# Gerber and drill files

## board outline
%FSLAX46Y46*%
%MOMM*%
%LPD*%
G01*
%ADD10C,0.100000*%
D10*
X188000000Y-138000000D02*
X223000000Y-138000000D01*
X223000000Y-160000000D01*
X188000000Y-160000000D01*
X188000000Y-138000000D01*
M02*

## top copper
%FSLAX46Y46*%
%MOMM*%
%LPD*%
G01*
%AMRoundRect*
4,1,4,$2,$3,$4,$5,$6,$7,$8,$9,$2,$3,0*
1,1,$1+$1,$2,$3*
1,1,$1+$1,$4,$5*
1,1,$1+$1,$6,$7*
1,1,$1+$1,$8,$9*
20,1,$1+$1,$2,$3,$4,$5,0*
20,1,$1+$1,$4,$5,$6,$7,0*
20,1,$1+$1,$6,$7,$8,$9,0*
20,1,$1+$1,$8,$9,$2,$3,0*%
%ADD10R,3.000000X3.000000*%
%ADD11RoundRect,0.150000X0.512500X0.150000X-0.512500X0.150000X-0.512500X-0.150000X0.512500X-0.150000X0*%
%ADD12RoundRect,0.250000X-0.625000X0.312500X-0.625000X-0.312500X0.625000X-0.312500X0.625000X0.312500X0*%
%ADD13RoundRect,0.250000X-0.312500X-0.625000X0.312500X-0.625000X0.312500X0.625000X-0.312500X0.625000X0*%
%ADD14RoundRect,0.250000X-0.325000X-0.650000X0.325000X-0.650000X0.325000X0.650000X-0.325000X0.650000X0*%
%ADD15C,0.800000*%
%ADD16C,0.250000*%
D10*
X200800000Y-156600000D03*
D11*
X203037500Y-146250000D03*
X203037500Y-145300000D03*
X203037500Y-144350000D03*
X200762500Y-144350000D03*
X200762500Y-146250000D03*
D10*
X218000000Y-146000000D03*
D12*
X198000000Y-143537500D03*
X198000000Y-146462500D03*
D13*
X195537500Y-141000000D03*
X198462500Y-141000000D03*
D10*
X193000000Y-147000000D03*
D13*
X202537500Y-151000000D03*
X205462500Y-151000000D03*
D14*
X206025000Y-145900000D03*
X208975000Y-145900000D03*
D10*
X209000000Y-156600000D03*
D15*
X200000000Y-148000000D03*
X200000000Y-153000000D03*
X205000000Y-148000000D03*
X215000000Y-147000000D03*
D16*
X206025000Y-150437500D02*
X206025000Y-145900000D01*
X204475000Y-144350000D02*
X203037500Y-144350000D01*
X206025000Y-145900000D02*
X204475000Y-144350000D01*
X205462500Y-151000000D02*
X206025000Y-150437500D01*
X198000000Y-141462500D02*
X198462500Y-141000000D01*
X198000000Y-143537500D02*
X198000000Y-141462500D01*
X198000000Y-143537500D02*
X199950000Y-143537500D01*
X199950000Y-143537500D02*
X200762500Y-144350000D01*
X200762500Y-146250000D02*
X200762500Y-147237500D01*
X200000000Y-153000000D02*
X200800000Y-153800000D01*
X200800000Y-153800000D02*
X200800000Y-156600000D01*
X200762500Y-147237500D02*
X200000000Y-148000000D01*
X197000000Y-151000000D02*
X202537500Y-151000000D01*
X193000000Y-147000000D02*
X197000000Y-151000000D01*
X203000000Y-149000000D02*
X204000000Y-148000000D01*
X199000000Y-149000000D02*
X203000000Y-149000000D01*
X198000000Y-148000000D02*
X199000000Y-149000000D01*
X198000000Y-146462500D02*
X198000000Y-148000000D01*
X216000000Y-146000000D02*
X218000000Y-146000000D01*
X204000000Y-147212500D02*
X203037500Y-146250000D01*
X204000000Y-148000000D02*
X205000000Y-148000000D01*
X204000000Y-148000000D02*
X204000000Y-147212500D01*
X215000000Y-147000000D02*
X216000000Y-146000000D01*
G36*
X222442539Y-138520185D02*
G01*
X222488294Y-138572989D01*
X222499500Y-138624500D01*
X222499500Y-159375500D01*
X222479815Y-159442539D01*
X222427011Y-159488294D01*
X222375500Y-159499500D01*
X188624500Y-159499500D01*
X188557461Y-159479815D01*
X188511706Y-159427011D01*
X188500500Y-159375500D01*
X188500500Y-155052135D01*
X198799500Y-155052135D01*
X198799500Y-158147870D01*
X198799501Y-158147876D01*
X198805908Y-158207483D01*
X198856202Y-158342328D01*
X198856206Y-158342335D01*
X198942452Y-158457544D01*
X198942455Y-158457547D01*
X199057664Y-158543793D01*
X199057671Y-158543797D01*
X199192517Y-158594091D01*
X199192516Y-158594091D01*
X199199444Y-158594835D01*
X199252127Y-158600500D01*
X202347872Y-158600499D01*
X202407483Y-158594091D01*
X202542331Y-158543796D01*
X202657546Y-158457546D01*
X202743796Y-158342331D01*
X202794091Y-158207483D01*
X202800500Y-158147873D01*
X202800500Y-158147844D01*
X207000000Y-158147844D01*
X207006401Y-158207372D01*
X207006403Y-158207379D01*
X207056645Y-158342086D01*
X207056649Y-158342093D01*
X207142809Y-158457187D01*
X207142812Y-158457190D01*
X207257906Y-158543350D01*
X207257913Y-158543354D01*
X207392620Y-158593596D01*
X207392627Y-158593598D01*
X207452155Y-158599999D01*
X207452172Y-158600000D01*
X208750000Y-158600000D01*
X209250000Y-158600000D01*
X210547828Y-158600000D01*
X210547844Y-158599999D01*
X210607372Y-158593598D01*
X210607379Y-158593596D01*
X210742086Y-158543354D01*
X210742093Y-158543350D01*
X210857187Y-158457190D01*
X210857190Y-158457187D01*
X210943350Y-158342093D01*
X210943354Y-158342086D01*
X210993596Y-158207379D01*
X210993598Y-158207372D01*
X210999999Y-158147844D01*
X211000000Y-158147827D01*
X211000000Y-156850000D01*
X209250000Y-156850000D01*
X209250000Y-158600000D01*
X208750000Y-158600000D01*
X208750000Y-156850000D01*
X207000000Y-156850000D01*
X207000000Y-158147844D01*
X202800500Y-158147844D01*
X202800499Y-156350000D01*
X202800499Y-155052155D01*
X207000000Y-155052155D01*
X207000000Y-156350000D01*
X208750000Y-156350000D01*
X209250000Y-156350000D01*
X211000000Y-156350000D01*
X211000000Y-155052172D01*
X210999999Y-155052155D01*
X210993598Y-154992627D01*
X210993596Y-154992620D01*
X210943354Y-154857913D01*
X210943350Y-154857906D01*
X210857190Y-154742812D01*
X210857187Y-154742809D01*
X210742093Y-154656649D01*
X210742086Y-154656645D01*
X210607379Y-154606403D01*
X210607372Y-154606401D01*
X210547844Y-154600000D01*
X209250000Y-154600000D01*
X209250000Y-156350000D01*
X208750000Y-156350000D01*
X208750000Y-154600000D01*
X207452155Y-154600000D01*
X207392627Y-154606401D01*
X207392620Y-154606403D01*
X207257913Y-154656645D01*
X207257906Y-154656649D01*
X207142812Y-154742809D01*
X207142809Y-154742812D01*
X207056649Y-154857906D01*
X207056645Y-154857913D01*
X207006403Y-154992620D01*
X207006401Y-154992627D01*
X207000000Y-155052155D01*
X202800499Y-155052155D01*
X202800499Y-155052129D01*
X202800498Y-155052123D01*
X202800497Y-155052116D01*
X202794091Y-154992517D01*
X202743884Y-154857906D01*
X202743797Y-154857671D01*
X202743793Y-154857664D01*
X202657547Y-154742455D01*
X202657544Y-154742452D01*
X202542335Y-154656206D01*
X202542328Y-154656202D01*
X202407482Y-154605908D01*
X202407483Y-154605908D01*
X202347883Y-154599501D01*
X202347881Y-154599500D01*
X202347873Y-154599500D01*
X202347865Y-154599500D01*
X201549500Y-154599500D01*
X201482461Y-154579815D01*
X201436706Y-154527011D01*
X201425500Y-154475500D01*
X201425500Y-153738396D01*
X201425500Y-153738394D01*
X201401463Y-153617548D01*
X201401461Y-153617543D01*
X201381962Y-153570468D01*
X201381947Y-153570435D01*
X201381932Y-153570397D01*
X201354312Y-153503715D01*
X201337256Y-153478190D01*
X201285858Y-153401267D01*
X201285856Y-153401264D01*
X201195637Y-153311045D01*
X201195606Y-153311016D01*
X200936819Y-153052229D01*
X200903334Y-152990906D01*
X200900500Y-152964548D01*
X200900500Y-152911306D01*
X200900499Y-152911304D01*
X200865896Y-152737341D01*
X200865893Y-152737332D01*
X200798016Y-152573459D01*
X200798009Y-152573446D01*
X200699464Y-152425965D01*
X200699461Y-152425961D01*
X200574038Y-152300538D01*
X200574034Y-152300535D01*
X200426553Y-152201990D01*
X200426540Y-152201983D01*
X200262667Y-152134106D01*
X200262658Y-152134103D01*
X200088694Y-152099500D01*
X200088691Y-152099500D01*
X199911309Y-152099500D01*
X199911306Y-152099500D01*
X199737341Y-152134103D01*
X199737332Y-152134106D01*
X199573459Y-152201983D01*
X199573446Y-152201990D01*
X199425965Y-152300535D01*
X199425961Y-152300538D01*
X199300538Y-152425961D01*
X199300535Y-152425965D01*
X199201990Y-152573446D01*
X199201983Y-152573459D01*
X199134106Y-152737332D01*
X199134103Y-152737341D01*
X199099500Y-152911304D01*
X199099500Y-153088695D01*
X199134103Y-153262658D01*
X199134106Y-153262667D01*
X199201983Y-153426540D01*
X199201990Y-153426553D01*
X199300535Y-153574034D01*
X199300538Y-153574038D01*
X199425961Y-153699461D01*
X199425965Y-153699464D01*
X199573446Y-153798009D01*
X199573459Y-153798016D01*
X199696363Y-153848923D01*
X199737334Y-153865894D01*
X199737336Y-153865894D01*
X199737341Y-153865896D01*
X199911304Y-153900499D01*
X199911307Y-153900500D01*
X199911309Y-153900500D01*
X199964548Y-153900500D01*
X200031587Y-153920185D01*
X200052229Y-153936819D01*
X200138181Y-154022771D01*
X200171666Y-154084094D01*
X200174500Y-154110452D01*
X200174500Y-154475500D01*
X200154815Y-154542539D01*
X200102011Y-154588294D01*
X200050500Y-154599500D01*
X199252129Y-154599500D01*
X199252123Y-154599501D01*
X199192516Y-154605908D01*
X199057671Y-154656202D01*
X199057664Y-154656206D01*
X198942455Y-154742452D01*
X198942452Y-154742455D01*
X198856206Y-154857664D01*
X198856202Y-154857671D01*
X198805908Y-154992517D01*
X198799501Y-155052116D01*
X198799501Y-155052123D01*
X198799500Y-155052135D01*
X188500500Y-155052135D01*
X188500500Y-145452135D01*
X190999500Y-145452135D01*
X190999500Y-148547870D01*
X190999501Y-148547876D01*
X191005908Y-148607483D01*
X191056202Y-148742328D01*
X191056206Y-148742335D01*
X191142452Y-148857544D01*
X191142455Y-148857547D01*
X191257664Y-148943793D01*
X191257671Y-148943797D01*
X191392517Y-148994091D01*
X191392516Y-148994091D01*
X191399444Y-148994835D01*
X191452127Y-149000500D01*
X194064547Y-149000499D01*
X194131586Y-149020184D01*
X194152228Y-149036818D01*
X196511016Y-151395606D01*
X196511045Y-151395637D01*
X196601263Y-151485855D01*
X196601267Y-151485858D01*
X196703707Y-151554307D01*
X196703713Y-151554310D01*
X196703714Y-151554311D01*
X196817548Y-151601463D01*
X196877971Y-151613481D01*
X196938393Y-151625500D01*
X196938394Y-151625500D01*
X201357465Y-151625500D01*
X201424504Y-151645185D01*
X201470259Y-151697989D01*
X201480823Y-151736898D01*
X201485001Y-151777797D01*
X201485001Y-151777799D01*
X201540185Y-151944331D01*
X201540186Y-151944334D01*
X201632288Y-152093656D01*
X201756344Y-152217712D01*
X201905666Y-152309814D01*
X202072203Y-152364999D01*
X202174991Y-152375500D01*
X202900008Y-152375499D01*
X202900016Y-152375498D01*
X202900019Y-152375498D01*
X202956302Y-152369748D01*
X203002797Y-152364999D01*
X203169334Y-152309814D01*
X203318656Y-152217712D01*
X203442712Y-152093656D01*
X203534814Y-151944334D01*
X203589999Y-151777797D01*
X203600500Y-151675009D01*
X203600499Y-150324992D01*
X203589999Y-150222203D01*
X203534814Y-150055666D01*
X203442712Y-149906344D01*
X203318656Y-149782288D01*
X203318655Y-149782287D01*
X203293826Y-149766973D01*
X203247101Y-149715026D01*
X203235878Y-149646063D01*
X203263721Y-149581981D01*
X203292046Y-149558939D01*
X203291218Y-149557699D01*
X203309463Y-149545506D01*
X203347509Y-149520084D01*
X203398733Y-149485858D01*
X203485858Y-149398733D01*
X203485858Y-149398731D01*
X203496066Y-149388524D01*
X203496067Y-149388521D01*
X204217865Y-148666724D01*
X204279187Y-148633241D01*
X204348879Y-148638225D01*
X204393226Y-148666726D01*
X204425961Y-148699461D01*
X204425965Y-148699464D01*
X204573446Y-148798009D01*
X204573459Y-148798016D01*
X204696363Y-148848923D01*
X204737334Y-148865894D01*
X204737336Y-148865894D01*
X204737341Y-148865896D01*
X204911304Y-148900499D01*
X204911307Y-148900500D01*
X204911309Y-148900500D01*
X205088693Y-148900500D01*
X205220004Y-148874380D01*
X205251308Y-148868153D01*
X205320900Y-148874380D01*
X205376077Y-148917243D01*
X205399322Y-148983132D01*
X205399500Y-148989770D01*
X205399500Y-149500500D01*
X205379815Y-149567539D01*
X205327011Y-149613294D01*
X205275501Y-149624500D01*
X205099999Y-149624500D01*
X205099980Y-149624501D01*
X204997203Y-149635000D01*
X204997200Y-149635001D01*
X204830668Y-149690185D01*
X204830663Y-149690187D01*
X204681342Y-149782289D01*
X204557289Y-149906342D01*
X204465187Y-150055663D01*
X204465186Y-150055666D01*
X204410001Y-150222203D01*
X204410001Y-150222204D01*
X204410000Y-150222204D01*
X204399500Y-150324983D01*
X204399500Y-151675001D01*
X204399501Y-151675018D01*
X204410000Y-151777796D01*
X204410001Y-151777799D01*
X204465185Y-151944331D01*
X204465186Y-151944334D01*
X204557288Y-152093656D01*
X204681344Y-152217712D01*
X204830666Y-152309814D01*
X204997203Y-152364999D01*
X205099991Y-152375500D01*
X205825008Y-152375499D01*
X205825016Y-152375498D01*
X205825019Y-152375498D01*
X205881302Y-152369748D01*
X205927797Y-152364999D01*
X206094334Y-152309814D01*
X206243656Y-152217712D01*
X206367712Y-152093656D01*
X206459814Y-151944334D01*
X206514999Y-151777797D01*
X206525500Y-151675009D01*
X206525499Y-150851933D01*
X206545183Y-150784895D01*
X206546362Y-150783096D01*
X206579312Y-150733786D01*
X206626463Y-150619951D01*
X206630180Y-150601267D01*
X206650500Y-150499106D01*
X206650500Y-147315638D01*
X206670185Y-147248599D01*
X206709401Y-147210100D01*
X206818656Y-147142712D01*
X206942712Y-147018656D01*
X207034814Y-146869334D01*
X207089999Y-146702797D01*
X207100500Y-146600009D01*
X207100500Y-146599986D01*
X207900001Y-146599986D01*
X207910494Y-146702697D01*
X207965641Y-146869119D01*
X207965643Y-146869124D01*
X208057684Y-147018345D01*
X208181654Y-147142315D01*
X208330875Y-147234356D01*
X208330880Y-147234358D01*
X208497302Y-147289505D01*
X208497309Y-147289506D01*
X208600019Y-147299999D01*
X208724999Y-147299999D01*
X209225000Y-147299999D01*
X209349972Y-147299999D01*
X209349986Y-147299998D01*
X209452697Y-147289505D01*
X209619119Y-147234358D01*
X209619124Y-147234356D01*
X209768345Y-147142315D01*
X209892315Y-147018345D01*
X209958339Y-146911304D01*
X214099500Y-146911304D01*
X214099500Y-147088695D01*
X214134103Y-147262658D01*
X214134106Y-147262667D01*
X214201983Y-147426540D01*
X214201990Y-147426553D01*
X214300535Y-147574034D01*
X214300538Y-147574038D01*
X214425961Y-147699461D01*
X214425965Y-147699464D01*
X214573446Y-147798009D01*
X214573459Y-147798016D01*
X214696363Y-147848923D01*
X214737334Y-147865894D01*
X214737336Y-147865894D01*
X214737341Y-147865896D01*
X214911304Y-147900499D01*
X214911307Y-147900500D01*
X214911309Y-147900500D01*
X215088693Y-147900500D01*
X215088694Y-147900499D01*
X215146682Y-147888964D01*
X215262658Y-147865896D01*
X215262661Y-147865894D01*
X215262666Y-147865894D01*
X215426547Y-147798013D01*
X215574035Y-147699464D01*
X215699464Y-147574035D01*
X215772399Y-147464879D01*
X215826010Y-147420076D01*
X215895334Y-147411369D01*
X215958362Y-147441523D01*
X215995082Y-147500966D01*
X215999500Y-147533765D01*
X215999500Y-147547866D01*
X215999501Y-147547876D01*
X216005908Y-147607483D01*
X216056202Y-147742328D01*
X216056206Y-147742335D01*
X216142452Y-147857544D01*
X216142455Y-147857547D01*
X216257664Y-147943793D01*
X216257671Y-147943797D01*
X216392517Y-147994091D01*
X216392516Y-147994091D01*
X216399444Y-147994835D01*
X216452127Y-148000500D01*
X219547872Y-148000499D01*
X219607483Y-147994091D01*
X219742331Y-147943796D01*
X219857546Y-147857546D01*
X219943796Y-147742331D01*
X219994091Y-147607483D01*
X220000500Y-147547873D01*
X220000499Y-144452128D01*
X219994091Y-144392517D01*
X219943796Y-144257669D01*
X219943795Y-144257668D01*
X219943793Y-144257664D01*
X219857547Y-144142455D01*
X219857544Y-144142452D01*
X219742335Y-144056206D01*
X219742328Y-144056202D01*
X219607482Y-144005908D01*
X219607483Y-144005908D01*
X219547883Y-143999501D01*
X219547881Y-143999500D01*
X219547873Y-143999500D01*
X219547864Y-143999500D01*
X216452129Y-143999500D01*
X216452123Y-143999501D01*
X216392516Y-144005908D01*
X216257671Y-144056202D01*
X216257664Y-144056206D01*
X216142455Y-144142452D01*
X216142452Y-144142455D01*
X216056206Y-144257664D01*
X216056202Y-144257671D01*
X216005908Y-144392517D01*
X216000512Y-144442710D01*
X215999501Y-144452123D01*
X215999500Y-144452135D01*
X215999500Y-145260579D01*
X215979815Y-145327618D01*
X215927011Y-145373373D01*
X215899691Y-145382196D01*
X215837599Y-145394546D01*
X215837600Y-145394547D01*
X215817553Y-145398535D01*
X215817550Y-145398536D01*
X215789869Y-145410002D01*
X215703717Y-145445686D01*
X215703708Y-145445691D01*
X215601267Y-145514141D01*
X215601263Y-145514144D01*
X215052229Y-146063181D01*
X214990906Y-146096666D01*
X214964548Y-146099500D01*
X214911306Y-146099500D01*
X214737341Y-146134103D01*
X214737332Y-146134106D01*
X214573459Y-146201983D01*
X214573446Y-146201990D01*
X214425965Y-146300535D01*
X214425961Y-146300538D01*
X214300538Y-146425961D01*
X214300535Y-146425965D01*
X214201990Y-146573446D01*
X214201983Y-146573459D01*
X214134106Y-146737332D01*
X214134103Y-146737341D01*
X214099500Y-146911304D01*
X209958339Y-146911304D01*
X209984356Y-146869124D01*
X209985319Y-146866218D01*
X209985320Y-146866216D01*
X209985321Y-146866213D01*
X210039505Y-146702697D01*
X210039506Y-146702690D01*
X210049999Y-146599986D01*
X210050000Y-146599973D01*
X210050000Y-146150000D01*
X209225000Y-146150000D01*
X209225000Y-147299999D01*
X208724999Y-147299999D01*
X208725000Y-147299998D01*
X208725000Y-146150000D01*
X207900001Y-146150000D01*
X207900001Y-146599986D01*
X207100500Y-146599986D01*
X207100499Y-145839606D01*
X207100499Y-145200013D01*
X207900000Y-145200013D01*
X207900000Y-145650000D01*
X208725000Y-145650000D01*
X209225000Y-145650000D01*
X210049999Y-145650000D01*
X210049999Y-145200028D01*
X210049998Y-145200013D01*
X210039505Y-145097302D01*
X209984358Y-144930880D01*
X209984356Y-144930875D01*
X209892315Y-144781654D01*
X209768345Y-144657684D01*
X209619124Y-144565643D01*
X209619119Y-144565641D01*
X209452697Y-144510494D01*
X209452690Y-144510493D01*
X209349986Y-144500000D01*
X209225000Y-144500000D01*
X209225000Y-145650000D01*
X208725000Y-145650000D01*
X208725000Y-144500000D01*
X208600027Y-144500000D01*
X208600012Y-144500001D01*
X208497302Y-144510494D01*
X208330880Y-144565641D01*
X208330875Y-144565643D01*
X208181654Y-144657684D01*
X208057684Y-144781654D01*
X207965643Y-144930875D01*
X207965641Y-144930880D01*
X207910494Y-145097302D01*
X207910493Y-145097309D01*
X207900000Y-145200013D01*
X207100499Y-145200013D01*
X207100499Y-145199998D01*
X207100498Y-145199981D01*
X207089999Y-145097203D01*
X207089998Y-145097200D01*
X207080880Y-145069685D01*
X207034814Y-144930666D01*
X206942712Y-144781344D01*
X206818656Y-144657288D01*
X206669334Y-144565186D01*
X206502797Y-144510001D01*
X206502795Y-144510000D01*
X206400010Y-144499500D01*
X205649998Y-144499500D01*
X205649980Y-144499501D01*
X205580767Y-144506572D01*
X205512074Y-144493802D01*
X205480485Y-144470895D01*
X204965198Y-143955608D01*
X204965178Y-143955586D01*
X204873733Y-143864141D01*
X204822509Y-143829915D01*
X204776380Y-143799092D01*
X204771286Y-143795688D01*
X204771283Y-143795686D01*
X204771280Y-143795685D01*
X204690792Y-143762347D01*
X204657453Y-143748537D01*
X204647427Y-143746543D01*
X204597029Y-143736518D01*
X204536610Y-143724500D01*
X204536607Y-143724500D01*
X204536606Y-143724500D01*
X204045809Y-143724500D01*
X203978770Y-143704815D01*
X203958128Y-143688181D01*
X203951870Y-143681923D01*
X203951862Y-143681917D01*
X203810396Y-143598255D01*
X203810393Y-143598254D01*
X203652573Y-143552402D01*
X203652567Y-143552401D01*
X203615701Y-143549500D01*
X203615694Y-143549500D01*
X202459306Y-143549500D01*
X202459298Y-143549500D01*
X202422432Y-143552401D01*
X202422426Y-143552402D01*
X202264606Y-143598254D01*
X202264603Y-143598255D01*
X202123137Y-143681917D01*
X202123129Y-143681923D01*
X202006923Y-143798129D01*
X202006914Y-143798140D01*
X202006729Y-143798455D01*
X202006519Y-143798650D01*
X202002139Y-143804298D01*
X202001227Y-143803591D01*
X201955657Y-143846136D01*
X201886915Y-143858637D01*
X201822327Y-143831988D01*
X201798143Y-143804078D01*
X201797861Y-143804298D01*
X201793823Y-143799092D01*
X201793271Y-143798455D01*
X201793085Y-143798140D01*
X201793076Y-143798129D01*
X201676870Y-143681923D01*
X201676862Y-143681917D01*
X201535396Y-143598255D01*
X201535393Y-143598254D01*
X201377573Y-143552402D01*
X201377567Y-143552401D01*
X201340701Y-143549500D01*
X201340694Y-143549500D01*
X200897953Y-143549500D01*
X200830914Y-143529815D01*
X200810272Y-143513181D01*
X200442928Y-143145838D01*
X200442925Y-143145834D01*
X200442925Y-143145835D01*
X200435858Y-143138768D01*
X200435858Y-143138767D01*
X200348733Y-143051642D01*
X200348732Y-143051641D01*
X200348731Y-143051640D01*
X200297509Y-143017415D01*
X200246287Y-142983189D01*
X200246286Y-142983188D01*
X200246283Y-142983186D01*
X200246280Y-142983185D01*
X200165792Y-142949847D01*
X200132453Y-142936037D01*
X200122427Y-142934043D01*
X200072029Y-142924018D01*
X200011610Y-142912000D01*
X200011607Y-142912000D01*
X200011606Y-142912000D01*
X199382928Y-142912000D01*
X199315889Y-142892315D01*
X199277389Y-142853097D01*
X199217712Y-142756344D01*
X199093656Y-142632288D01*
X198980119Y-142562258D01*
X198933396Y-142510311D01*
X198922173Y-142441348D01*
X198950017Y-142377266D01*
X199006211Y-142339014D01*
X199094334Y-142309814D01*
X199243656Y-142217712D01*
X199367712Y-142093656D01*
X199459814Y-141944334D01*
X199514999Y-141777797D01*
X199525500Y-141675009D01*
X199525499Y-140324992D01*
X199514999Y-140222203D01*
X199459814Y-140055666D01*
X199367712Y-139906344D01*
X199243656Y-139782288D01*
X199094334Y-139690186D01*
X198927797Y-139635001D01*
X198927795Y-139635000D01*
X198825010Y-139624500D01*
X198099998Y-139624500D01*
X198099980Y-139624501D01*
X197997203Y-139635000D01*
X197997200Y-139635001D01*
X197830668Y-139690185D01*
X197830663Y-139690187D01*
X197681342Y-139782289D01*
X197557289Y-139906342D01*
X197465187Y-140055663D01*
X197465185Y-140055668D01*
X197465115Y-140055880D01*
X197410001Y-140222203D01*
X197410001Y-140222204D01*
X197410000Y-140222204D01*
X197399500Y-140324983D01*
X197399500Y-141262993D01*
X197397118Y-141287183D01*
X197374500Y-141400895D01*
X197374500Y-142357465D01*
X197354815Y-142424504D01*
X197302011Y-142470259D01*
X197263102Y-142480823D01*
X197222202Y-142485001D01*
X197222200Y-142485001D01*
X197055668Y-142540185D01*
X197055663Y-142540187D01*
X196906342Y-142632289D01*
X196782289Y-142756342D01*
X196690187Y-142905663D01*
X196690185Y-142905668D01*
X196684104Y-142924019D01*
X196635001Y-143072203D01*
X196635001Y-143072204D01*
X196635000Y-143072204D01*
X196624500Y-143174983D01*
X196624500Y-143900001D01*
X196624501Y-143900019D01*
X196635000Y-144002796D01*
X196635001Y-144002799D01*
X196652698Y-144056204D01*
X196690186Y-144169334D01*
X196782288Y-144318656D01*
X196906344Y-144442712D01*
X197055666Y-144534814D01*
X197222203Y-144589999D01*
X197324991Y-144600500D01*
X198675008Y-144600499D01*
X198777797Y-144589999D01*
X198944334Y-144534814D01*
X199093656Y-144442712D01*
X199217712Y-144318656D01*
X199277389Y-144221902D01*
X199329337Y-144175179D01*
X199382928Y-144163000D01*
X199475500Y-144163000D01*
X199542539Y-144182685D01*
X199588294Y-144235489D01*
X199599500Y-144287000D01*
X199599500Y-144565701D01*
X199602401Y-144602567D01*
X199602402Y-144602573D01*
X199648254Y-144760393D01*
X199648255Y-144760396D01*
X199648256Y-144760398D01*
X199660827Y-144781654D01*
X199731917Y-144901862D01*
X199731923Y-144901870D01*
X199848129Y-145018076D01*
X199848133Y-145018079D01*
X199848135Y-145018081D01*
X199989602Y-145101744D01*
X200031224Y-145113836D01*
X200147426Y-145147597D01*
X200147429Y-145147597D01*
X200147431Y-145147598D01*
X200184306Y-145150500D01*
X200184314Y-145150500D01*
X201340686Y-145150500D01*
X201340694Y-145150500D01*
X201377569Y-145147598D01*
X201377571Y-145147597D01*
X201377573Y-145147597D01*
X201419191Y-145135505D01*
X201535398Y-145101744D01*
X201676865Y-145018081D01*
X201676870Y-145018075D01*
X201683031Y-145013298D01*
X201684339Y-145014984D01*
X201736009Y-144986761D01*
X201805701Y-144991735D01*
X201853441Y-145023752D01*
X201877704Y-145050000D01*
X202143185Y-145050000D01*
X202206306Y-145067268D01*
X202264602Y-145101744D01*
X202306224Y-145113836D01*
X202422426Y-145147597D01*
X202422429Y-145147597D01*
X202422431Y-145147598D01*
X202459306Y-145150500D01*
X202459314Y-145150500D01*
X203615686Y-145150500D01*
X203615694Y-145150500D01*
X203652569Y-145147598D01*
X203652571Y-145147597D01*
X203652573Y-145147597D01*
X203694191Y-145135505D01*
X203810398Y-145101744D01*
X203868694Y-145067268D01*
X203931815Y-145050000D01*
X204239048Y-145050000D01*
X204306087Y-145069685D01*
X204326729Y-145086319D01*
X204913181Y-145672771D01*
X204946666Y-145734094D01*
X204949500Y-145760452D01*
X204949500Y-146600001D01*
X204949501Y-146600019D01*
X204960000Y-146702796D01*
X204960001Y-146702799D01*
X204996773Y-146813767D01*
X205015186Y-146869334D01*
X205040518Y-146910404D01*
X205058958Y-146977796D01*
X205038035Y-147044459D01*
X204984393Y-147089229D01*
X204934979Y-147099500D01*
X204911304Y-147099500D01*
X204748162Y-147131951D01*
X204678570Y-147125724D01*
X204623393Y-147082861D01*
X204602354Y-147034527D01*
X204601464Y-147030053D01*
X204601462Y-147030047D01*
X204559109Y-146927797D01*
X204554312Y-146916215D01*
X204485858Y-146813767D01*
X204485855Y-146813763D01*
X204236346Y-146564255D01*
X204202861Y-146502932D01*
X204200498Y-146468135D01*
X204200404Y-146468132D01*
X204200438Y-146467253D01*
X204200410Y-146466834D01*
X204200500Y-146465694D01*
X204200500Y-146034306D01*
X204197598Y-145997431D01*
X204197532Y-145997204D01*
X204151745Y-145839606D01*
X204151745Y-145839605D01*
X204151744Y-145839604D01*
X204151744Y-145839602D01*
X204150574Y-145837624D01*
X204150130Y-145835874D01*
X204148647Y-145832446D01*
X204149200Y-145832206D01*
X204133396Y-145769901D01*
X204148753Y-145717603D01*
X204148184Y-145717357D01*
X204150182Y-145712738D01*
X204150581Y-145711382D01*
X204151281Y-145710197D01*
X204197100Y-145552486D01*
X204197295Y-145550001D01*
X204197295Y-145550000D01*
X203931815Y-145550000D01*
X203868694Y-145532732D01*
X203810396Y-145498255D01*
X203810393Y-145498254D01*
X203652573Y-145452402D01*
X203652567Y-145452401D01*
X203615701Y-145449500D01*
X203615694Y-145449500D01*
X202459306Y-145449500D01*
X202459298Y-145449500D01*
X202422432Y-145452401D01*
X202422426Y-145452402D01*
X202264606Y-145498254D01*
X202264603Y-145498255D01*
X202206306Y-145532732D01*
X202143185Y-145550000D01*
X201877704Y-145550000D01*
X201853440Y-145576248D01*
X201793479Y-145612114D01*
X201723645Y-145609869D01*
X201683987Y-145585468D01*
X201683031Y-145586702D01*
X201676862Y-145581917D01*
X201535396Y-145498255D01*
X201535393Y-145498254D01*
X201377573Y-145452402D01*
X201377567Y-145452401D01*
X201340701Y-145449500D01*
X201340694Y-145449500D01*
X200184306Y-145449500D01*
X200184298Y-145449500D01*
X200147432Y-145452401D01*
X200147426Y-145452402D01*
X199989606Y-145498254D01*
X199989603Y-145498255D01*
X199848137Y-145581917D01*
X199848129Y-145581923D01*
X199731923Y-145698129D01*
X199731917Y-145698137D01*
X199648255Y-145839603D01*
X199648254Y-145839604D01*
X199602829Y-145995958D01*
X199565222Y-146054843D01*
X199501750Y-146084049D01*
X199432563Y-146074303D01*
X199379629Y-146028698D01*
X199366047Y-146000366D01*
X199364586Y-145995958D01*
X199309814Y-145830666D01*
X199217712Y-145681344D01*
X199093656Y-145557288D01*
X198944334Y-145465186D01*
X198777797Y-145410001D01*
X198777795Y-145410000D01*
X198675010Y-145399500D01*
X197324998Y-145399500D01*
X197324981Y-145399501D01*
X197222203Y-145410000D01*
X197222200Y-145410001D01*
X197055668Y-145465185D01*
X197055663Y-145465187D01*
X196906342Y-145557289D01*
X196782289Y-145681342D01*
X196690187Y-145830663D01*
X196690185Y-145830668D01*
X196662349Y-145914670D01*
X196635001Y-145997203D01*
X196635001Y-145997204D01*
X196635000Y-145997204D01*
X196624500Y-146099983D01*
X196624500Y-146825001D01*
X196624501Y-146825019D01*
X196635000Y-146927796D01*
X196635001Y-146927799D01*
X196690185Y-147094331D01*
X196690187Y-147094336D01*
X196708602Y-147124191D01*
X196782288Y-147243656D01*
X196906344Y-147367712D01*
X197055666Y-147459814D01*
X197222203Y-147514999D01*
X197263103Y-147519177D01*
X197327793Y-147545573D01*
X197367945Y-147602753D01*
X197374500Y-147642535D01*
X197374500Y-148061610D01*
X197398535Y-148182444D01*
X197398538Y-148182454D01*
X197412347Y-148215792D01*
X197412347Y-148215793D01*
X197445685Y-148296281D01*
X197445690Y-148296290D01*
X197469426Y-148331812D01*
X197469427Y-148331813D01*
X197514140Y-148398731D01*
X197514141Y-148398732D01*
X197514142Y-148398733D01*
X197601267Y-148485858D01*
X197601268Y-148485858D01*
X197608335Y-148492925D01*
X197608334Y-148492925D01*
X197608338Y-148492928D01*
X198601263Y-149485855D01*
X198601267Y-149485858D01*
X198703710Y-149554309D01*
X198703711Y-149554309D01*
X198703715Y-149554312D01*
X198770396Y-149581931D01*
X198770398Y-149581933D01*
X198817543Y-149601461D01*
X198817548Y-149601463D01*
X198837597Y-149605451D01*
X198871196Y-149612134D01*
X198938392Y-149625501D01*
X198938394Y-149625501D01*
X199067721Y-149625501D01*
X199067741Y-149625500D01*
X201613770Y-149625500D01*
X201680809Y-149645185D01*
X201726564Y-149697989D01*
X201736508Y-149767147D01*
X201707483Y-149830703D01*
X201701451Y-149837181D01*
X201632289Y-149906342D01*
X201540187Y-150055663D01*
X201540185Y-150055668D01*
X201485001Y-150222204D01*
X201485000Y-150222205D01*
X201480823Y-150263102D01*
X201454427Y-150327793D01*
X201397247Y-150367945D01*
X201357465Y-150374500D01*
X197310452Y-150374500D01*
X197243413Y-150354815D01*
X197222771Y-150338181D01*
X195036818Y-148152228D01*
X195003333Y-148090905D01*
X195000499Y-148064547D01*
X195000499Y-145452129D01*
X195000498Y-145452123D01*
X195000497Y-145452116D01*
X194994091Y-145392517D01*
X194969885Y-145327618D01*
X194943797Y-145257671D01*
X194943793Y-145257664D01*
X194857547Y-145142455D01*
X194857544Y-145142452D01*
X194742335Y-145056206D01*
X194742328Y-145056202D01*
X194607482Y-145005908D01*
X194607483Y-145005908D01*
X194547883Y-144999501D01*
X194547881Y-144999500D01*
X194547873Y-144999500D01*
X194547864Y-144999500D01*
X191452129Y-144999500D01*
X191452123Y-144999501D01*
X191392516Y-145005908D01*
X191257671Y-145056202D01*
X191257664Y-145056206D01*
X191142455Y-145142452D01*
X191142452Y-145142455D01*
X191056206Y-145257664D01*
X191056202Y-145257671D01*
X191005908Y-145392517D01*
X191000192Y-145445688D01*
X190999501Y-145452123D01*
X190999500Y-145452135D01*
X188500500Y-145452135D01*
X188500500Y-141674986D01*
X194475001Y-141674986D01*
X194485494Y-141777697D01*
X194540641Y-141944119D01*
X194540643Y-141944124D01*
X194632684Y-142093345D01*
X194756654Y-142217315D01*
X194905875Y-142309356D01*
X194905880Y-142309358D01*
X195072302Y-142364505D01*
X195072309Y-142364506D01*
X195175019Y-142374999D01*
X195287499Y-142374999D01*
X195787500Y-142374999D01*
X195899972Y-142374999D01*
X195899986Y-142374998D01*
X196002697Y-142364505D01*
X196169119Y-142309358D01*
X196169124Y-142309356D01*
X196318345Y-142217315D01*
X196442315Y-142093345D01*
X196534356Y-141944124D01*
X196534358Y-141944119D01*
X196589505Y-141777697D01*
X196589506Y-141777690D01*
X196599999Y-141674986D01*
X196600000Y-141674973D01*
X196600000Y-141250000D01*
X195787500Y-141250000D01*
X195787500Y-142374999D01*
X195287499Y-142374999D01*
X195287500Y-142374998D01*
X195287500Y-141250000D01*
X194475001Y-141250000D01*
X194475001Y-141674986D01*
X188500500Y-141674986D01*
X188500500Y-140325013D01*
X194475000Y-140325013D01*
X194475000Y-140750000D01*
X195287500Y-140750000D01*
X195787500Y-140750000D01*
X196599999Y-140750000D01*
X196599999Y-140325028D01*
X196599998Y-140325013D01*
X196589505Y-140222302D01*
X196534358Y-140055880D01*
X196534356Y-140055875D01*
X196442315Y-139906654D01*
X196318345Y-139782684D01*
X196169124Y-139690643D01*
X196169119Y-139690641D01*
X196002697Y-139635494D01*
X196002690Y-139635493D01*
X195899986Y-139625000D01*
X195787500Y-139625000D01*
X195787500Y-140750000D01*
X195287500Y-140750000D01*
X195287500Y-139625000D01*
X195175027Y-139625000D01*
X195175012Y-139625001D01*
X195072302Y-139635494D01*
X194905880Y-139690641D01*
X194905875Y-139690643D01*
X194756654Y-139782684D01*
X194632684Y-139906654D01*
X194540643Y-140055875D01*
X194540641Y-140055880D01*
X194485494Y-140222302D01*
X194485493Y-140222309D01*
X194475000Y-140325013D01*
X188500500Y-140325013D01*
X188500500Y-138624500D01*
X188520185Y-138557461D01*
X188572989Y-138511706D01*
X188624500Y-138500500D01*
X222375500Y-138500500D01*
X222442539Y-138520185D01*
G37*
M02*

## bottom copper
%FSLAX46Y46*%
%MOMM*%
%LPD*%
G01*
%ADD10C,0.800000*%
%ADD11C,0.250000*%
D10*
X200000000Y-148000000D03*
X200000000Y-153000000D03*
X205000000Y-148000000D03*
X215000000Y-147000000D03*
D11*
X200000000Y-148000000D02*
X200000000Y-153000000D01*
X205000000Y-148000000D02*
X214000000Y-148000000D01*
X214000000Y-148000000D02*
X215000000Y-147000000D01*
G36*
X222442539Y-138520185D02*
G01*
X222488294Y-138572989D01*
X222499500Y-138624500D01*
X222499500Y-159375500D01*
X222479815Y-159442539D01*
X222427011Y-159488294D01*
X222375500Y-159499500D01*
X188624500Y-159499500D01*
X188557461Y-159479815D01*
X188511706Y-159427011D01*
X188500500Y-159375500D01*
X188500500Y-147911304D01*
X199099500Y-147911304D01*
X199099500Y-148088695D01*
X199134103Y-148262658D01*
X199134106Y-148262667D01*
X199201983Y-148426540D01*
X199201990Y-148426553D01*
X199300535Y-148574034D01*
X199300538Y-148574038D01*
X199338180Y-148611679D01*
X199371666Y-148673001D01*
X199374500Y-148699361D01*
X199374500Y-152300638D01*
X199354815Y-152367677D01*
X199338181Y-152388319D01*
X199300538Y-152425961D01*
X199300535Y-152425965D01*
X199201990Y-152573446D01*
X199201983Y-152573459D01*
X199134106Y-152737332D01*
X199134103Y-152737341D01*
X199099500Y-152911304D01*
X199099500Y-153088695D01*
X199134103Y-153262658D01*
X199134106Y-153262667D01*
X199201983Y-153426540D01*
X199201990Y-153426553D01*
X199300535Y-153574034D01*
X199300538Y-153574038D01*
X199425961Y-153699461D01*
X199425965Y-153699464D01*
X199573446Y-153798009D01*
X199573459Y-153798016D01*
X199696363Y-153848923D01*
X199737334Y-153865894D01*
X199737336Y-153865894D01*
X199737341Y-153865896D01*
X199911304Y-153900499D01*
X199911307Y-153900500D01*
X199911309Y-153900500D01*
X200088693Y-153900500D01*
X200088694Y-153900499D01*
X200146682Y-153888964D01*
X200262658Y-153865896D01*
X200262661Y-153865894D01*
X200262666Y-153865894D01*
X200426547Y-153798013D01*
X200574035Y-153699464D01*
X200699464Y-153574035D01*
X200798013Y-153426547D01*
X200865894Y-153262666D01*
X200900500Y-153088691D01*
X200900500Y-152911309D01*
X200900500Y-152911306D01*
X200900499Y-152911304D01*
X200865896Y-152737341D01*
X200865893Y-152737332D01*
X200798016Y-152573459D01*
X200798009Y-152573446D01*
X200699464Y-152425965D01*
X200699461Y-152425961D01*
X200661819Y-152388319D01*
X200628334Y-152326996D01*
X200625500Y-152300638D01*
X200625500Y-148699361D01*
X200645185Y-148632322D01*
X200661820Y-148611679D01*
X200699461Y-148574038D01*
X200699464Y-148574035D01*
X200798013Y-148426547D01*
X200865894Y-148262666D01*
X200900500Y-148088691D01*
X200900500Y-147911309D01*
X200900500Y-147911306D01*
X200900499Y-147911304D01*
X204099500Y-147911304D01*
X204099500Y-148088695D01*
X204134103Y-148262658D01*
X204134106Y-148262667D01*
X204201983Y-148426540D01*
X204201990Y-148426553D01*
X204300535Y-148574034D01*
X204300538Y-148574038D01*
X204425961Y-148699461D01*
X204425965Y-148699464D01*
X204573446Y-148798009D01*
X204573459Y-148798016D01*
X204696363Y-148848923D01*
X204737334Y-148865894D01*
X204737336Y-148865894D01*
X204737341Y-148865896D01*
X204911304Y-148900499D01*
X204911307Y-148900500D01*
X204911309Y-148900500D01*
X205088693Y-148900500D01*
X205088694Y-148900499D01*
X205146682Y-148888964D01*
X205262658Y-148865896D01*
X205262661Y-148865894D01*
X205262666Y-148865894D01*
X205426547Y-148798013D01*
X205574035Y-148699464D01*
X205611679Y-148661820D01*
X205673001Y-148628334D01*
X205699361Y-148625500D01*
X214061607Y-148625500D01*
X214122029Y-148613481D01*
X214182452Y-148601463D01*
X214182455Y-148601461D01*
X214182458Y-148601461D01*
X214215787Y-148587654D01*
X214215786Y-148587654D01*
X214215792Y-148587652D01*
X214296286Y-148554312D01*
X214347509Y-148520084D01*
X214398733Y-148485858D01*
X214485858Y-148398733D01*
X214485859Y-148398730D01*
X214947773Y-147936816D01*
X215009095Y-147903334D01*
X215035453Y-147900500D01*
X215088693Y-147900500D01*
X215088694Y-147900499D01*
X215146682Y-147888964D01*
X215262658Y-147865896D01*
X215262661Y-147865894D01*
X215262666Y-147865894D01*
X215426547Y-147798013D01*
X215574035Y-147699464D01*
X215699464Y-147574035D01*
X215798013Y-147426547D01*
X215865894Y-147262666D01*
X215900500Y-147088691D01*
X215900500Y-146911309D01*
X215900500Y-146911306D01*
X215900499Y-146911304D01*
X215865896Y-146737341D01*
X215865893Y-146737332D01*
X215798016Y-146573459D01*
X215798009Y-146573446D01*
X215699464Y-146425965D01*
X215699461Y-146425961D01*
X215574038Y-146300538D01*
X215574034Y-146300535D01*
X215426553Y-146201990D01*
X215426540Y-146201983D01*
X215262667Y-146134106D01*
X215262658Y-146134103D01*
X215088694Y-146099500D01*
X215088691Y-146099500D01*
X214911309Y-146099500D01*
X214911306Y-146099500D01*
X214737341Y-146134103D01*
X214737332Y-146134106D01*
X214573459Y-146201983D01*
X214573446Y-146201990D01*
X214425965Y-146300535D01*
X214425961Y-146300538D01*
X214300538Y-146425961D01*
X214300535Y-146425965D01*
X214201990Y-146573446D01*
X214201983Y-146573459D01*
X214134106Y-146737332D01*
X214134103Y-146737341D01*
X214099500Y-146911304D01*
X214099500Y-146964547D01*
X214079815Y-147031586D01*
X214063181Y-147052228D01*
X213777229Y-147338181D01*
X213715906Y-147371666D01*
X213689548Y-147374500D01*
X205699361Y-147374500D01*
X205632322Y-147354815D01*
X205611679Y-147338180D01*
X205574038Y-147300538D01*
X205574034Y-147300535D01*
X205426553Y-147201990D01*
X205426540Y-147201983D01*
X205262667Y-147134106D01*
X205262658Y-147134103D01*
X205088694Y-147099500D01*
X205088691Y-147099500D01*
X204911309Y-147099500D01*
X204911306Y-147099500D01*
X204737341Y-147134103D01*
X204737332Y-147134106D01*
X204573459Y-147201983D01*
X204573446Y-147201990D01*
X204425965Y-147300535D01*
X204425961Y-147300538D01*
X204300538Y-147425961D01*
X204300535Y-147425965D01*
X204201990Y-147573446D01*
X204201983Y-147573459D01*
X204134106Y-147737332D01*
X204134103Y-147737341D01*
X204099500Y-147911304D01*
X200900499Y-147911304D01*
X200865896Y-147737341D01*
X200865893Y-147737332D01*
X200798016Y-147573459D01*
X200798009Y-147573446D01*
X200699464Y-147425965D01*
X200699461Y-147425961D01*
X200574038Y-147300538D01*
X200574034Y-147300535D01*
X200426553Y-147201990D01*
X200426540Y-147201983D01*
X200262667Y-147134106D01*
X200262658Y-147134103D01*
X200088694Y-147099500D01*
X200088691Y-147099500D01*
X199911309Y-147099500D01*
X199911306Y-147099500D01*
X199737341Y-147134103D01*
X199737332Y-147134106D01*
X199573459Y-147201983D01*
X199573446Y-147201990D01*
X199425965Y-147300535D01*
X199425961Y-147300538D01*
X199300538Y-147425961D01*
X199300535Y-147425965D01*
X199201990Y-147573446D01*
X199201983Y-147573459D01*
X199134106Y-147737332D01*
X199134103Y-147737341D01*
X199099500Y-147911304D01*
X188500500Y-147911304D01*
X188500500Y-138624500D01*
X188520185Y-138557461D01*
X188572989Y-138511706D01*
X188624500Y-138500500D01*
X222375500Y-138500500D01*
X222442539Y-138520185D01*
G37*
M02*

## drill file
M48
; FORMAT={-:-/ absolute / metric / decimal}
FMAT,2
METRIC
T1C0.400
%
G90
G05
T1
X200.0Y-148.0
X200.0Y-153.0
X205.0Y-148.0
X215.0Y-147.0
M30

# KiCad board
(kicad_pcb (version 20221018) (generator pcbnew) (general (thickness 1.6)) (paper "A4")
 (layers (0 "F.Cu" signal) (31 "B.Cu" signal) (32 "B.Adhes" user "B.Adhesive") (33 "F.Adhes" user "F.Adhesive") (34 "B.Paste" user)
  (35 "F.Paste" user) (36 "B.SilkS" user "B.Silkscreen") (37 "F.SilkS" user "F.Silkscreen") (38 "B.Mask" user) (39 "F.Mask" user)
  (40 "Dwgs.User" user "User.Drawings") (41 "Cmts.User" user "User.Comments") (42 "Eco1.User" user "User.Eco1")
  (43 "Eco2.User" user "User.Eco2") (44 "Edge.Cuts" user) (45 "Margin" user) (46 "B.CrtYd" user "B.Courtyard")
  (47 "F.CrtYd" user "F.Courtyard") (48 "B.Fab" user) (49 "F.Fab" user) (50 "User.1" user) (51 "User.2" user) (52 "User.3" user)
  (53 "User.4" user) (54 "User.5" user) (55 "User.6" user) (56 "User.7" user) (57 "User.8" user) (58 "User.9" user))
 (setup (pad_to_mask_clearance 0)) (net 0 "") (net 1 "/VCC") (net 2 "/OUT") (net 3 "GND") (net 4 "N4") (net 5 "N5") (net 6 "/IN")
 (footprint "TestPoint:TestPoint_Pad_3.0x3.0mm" (layer "F.Cu") (at 200.8 156.6)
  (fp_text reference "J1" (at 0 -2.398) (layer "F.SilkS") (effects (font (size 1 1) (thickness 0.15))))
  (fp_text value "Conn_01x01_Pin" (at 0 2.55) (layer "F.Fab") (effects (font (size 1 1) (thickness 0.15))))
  (pad "1" smd rect (at 0 0) (size 3 3) (layers "F.Cu" "F.Mask") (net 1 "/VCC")))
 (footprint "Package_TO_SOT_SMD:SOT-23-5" (layer "F.Cu") (at 201.9 145.3 180)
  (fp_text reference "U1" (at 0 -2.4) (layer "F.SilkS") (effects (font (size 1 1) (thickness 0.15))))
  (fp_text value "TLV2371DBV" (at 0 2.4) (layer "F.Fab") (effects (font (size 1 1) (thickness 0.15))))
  (pad "1" smd roundrect (at -1.1375 -0.95 180) (size 1.325 0.6) (layers "F.Cu" "F.Paste" "F.Mask") (roundrect_rratio 0.25) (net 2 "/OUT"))
  (pad "2" smd roundrect (at -1.1375 0 180) (size 1.325 0.6) (layers "F.Cu" "F.Paste" "F.Mask") (roundrect_rratio 0.25) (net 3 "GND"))
  (pad "3" smd roundrect (at -1.1375 0.95 180) (size 1.325 0.6) (layers "F.Cu" "F.Paste" "F.Mask") (roundrect_rratio 0.25) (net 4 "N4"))
  (pad "4" smd roundrect (at 1.1375 0.95 180) (size 1.325 0.6) (layers "F.Cu" "F.Paste" "F.Mask") (roundrect_rratio 0.25) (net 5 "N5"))
  (pad "5" smd roundrect (at 1.1375 -0.95 180) (size 1.325 0.6) (layers "F.Cu" "F.Paste" "F.Mask") (roundrect_rratio 0.25) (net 1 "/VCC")))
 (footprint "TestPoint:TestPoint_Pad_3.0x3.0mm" (layer "F.Cu") (at 218 146)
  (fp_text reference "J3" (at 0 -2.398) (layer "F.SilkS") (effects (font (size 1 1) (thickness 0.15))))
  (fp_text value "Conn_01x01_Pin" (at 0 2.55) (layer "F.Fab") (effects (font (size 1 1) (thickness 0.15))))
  (pad "1" smd rect (at 0 0) (size 3 3) (layers "F.Cu" "F.Mask") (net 2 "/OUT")))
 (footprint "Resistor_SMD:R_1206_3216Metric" (layer "F.Cu") (at 198 145 -90)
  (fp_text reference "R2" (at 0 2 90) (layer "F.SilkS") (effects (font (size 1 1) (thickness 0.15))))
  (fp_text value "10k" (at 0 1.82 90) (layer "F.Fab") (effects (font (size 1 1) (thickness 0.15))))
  (pad "1" smd roundrect (at -1.4625 0 270) (size 1.125 1.75) (layers "F.Cu" "F.Paste" "F.Mask") (roundrect_rratio 0.222222) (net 5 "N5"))
  (pad "2" smd roundrect (at 1.4625 0 270) (size 1.125 1.75) (layers "F.Cu" "F.Paste" "F.Mask") (roundrect_rratio 0.222222) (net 2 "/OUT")))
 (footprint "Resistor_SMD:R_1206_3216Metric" (layer "F.Cu") (at 197 141)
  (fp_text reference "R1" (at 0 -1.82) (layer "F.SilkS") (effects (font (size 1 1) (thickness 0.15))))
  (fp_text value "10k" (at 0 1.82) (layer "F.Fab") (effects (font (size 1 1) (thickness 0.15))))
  (pad "1" smd roundrect (at -1.4625 0) (size 1.125 1.75) (layers "F.Cu" "F.Paste" "F.Mask") (roundrect_rratio 0.222222) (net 3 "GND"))
  (pad "2" smd roundrect (at 1.4625 0) (size 1.125 1.75) (layers "F.Cu" "F.Paste" "F.Mask") (roundrect_rratio 0.222222) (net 5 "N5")))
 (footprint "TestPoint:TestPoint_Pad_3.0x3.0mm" (layer "F.Cu") (at 193 147)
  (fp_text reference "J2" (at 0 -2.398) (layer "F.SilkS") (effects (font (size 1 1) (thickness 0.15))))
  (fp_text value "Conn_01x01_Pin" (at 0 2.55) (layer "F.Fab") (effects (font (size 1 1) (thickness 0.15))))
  (pad "1" smd rect (at 0 0) (size 3 3) (layers "F.Cu" "F.Mask") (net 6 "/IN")))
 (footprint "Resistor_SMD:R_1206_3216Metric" (layer "F.Cu") (at 204 151)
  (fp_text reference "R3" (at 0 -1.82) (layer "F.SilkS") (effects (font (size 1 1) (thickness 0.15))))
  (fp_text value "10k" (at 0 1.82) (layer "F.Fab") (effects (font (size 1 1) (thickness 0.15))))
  (pad "1" smd roundrect (at -1.4625 0) (size 1.125 1.75) (layers "F.Cu" "F.Paste" "F.Mask") (roundrect_rratio 0.222222) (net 6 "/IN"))
  (pad "2" smd roundrect (at 1.4625 0) (size 1.125 1.75) (layers "F.Cu" "F.Paste" "F.Mask") (roundrect_rratio 0.222222) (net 4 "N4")))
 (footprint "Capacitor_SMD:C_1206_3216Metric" (layer "F.Cu") (at 207.5 145.9)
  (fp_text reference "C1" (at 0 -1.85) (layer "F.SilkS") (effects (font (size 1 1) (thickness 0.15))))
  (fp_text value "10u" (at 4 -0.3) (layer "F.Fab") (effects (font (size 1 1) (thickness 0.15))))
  (pad "1" smd roundrect (at -1.475 0) (size 1.15 1.8) (layers "F.Cu" "F.Paste" "F.Mask") (roundrect_rratio 0.217391) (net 4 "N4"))
  (pad "2" smd roundrect (at 1.475 0) (size 1.15 1.8) (layers "F.Cu" "F.Paste" "F.Mask") (roundrect_rratio 0.217391) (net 3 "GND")))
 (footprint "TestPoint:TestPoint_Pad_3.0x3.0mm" (layer "F.Cu") (at 209 156.6)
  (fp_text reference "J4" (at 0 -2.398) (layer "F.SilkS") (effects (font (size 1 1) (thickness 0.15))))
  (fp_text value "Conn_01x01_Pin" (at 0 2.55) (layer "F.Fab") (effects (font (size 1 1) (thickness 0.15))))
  (pad "1" smd rect (at 0 0) (size 3 3) (layers "F.Cu" "F.Mask") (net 3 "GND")))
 (gr_rect (start 188 138) (end 223 160) (stroke (width 0.1) (type default)) (fill none) (layer "Edge.Cuts"))
 (segment (start 206.025 150.4375) (end 206.025 145.9) (width 0.25) (layer "F.Cu") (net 4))
 (segment (start 204.475 144.35) (end 203.0375 144.35) (width 0.25) (layer "F.Cu") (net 4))
 (segment (start 206.025 145.9) (end 204.475 144.35) (width 0.25) (layer "F.Cu") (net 4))
 (segment (start 205.4625 151) (end 206.025 150.4375) (width 0.25) (layer "F.Cu") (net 4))
 (segment (start 198 141.4625) (end 198.4625 141) (width 0.25) (layer "F.Cu") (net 5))
 (segment (start 198 143.5375) (end 198 141.4625) (width 0.25) (layer "F.Cu") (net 5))
 (segment (start 198 143.5375) (end 199.95 143.5375) (width 0.25) (layer "F.Cu") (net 5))
 (segment (start 199.95 143.5375) (end 200.7625 144.35) (width 0.25) (layer "F.Cu") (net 5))
 (segment (start 200.7625 146.25) (end 200.7625 147.2375) (width 0.25) (layer "F.Cu") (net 1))
 (segment (start 200 153) (end 200.8 153.8) (width 0.25) (layer "F.Cu") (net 1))
 (segment (start 200.8 153.8) (end 200.8 156.6) (width 0.25) (layer "F.Cu") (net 1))
 (segment (start 200.7625 147.2375) (end 200 148) (width 0.25) (layer "F.Cu") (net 1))
 (via (at 200 148) (size 0.8) (drill 0.4) (layers "F.Cu" "B.Cu") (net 1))
 (via (at 200 153) (size 0.8) (drill 0.4) (layers "F.Cu" "B.Cu") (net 1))
 (segment (start 200 148) (end 200 153) (width 0.25) (layer "B.Cu") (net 1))
 (segment (start 197 151) (end 202.5375 151) (width 0.25) (layer "F.Cu") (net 6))
 (segment (start 193 147) (end 197 151) (width 0.25) (layer "F.Cu") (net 6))
 (segment (start 203 149) (end 204 148) (width 0.25) (layer "F.Cu") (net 2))
 (segment (start 199 149) (end 203 149) (width 0.25) (layer "F.Cu") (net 2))
 (segment (start 198 148) (end 199 149) (width 0.25) (layer "F.Cu") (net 2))
 (segment (start 198 146.4625) (end 198 148) (width 0.25) (layer "F.Cu") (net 2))
 (segment (start 216 146) (end 218 146) (width 0.25) (layer "F.Cu") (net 2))
 (segment (start 204 147.2125) (end 203.0375 146.25) (width 0.25) (layer "F.Cu") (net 2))
 (segment (start 204 148) (end 205 148) (width 0.25) (layer "F.Cu") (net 2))
 (segment (start 204 148) (end 204 147.2125) (width 0.25) (layer "F.Cu") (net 2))
 (segment (start 215 147) (end 216 146) (width 0.25) (layer "F.Cu") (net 2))
 (via (at 205 148) (size 0.8) (drill 0.4) (layers "F.Cu" "B.Cu") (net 2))
 (via (at 215 147) (size 0.8) (drill 0.4) (layers "F.Cu" "B.Cu") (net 2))
 (segment (start 205 148) (end 214 148) (width 0.25) (layer "B.Cu") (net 2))
 (segment (start 214 148) (end 215 147) (width 0.25) (layer "B.Cu") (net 2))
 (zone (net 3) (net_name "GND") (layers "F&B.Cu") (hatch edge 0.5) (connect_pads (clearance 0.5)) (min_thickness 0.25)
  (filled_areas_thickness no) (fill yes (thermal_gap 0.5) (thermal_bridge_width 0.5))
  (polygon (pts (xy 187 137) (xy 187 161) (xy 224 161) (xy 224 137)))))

